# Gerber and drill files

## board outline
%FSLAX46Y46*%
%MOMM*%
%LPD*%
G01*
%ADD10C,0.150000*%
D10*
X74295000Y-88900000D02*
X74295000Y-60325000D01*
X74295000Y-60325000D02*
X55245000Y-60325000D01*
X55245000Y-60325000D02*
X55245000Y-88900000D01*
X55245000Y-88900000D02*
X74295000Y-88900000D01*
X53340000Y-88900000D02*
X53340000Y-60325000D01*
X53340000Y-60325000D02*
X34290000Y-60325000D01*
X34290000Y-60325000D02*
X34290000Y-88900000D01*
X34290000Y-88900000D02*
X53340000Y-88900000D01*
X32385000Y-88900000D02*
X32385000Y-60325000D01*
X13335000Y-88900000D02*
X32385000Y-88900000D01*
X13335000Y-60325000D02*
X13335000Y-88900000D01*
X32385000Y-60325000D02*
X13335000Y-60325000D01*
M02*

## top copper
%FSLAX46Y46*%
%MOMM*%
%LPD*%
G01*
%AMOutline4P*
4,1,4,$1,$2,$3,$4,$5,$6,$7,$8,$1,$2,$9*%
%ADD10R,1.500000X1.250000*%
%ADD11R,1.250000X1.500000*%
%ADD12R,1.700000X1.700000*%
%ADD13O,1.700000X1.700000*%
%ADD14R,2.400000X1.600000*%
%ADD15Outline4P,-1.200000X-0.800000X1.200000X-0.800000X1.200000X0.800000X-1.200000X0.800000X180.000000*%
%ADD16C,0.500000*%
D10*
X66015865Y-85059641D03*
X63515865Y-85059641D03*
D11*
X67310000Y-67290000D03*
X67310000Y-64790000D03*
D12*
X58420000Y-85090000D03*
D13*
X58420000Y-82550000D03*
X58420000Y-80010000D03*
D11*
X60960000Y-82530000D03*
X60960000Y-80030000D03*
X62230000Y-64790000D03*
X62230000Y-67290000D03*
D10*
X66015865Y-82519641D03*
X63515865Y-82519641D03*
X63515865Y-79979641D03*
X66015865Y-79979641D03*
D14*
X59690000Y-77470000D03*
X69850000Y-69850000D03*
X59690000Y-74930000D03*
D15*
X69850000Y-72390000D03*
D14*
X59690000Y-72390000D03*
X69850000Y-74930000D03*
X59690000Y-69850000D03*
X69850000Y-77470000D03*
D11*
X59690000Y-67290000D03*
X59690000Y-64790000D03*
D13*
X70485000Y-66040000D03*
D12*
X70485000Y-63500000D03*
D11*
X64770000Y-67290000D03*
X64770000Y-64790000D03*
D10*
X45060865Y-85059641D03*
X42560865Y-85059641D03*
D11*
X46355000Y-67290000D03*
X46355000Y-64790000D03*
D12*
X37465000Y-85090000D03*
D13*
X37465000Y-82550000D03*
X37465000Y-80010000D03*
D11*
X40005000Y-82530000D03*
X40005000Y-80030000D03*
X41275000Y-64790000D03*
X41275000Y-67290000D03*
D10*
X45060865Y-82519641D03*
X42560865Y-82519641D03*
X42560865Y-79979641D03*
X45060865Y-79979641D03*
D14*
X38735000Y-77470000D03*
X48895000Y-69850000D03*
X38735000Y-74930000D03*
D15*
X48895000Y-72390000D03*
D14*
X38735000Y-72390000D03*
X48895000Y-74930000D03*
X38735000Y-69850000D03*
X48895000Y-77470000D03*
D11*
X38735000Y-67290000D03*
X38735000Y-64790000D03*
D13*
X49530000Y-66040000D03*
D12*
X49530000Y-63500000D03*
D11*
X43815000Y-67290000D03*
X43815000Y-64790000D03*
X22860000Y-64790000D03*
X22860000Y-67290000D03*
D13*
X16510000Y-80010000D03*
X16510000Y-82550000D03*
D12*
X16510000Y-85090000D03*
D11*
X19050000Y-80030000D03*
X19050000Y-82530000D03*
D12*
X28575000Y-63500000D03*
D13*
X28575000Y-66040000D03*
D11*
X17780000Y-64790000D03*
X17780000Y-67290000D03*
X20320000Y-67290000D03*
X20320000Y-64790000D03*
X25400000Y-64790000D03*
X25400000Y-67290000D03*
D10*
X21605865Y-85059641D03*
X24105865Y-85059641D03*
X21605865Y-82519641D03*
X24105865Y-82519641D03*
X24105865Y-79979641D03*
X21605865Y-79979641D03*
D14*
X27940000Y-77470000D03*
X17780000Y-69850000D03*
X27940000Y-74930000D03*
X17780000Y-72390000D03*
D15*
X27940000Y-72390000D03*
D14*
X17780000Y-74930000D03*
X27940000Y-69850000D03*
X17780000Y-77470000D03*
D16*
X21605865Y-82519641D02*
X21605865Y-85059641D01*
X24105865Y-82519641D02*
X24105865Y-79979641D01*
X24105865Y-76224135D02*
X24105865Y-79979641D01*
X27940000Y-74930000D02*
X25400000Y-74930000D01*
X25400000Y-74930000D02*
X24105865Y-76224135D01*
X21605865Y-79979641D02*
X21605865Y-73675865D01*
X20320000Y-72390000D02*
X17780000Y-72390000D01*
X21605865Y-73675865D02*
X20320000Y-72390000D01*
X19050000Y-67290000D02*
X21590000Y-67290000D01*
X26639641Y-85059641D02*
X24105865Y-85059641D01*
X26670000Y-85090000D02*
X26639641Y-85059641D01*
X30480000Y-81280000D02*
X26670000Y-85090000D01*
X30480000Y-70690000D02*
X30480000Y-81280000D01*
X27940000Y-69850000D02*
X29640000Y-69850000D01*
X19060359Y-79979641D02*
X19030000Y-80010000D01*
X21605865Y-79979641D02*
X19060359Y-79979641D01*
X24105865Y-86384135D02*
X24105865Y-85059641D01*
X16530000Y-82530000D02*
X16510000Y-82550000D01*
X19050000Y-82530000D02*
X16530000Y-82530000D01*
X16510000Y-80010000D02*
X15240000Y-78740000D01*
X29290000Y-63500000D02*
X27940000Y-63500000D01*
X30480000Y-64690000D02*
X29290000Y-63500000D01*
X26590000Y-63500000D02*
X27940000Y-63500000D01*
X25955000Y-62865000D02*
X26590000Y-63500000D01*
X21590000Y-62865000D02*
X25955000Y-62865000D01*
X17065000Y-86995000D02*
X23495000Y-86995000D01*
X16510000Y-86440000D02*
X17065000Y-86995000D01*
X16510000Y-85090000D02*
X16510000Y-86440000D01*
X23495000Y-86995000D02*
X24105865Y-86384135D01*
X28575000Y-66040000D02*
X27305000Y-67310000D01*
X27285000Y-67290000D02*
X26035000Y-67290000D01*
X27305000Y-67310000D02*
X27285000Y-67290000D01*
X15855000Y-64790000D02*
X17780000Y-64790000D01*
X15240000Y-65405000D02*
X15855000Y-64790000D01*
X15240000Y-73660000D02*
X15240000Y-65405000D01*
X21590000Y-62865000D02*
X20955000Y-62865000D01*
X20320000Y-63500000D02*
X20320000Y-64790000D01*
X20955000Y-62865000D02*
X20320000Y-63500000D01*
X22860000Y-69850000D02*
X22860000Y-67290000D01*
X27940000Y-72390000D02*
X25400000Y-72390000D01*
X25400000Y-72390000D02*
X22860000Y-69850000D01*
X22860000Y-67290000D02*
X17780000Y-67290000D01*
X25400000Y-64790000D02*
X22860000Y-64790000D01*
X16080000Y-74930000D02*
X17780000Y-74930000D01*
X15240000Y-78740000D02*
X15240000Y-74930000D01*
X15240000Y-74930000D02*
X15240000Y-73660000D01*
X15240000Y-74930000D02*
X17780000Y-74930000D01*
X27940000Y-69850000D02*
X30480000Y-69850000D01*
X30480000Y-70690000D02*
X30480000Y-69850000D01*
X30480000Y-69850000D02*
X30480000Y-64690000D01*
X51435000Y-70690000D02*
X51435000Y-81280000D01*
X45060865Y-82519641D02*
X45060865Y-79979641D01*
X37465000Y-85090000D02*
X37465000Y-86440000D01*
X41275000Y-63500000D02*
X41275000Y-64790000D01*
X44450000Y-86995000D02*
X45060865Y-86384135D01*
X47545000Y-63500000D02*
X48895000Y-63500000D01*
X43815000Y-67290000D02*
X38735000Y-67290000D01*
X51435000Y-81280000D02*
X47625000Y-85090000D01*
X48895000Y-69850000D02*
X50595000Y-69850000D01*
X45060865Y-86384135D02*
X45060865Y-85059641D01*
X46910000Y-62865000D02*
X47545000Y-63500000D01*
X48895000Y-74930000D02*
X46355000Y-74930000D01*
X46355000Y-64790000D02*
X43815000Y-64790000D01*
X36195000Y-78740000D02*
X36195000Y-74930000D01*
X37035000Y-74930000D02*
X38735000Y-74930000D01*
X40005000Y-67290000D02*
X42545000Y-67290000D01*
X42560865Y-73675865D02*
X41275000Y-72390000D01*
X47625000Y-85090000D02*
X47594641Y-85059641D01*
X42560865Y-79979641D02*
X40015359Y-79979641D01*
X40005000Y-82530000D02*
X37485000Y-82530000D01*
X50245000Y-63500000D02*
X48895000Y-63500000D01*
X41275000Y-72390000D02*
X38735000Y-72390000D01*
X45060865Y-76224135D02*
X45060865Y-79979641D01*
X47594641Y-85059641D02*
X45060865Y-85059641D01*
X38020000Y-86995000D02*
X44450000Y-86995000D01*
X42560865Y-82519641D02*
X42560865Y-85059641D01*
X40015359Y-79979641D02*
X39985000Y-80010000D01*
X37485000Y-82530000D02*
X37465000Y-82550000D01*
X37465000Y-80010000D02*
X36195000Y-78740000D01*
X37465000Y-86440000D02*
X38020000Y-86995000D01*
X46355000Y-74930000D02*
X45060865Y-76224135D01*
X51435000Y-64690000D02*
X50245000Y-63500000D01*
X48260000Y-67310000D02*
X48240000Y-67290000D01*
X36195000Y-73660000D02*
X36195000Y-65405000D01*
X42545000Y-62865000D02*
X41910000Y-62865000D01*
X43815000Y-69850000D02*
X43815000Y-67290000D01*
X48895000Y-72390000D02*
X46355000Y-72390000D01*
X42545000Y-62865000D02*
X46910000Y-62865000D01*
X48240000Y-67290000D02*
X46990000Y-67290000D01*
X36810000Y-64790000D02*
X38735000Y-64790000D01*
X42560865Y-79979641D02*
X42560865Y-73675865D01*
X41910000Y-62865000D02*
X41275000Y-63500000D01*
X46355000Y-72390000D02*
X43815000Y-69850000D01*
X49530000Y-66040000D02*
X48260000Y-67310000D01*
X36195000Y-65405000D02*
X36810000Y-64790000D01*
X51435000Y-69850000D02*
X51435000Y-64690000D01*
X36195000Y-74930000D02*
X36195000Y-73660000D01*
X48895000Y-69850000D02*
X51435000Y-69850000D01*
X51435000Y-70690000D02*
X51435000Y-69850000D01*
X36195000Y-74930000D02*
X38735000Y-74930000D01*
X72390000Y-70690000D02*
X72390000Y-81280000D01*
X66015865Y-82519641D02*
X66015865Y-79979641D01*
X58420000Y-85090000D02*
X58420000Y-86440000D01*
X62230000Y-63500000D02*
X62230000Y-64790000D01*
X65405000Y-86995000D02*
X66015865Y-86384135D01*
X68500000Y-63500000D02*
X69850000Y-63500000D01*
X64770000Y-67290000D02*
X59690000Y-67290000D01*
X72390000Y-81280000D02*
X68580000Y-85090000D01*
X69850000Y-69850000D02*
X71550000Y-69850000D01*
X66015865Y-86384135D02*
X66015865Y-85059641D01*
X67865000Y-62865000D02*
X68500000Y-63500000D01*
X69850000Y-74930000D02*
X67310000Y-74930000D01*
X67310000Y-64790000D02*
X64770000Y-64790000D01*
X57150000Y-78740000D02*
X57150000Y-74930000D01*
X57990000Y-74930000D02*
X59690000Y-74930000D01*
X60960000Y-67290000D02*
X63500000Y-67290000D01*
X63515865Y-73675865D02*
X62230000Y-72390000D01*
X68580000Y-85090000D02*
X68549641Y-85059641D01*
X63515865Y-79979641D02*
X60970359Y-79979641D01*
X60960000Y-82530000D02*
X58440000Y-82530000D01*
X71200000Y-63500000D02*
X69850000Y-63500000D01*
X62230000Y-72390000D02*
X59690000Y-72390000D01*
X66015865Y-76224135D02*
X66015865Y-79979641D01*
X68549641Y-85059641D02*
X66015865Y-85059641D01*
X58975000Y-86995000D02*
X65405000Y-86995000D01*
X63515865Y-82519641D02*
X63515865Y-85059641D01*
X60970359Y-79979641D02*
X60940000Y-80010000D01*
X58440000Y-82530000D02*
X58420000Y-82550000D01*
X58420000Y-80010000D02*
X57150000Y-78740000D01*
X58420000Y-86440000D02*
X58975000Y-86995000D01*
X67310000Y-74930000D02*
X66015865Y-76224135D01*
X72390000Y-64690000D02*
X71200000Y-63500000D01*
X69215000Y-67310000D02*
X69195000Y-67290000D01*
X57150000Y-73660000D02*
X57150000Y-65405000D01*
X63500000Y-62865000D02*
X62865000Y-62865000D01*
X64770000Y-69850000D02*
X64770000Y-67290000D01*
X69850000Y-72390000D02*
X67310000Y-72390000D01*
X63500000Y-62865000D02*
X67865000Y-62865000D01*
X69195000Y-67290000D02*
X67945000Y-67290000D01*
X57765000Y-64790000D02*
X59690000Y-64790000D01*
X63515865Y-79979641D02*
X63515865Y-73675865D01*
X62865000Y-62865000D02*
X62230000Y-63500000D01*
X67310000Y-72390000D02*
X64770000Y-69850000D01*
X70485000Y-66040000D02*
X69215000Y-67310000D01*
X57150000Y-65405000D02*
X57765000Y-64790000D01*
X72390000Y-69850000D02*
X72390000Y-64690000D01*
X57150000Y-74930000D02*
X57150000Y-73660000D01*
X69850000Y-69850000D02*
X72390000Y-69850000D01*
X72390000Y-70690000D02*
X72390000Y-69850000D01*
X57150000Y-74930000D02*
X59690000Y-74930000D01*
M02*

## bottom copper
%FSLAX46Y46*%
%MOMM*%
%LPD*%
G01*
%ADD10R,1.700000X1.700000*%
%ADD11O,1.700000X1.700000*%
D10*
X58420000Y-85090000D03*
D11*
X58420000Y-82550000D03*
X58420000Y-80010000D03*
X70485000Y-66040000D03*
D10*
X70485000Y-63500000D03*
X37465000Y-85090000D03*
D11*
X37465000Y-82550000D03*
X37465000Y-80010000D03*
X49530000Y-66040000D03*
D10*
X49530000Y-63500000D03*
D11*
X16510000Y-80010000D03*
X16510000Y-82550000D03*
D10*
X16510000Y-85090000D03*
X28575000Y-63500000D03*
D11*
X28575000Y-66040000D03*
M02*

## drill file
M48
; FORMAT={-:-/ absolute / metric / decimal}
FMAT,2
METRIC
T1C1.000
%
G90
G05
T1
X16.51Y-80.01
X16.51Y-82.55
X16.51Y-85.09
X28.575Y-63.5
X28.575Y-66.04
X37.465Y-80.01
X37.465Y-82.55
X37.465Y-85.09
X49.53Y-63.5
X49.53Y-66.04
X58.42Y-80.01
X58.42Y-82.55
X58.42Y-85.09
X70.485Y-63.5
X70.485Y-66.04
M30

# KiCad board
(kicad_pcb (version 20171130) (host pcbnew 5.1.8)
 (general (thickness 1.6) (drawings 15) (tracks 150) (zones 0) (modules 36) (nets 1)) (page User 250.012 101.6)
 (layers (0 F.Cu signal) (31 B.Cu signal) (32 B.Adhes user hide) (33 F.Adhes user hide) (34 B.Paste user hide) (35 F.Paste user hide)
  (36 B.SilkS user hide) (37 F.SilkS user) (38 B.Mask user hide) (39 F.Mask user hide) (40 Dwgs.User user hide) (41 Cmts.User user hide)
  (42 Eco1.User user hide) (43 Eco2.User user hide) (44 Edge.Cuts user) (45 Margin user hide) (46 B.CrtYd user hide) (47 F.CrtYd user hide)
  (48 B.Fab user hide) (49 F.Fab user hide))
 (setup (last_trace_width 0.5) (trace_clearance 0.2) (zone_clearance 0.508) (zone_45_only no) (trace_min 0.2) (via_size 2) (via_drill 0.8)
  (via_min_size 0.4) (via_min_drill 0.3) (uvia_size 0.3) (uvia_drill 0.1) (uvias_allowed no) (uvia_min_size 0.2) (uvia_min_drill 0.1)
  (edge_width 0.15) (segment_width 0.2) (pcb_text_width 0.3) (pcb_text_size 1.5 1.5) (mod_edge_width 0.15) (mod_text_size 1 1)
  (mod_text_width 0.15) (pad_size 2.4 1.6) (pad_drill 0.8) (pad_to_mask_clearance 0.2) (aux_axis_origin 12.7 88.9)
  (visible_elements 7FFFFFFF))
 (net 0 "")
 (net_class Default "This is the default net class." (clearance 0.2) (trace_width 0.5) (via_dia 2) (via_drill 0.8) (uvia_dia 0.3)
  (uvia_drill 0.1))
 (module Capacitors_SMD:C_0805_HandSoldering (layer F.Cu) (at 64.765865 85.059641 180)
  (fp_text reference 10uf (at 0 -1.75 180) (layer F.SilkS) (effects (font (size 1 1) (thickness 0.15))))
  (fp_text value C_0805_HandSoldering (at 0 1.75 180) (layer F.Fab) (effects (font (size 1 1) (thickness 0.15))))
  (pad 1 smd rect (at -1.25 0 180) (size 1.5 1.25) (layers F.Cu F.Paste F.Mask))
  (pad 2 smd rect (at 1.25 0 180) (size 1.5 1.25) (layers F.Cu F.Paste F.Mask)))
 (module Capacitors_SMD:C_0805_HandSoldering (layer F.Cu) (at 67.31 66.04 270)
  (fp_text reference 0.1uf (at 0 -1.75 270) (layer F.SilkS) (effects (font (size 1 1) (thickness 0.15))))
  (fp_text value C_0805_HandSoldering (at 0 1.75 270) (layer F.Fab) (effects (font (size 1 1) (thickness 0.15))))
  (pad 2 smd rect (at 1.25 0 270) (size 1.5 1.25) (layers F.Cu F.Paste F.Mask))
  (pad 1 smd rect (at -1.25 0 270) (size 1.5 1.25) (layers F.Cu F.Paste F.Mask)))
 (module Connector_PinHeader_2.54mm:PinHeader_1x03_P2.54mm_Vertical (layer F.Cu) (at 58.42 85.09 180)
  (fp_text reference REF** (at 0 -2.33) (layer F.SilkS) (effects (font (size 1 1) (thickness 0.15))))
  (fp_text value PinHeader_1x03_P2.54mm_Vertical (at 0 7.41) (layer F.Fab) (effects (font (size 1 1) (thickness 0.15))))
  (pad 1 thru_hole rect (at 0 0 180) (size 1.7 1.7) (drill 1) (layers *.Cu *.Mask))
  (pad 2 thru_hole oval (at 0 2.54 180) (size 1.7 1.7) (drill 1) (layers *.Cu *.Mask))
  (pad 3 thru_hole oval (at 0 5.08 180) (size 1.7 1.7) (drill 1) (layers *.Cu *.Mask)))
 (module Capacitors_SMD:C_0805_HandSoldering (layer F.Cu) (at 60.96 81.28 270)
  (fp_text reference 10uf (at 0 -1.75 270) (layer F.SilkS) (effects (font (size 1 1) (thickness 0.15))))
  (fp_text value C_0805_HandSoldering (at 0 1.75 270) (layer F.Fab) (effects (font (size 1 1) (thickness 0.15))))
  (pad 2 smd rect (at 1.25 0 270) (size 1.5 1.25) (layers F.Cu F.Paste F.Mask))
  (pad 1 smd rect (at -1.25 0 270) (size 1.5 1.25) (layers F.Cu F.Paste F.Mask)))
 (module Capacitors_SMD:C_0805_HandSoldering (layer F.Cu) (at 62.23 66.04 270)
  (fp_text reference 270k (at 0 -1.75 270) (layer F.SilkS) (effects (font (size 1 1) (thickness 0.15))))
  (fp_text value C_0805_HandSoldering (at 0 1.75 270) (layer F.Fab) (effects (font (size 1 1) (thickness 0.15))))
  (pad 1 smd rect (at -1.25 0 270) (size 1.5 1.25) (layers F.Cu F.Paste F.Mask))
  (pad 2 smd rect (at 1.25 0 270) (size 1.5 1.25) (layers F.Cu F.Paste F.Mask)))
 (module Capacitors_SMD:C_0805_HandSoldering (layer F.Cu) (at 64.765865 82.519641 180)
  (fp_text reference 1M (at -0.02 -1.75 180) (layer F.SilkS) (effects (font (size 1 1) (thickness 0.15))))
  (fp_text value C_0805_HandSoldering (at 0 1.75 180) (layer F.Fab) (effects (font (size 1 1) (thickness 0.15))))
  (pad 1 smd rect (at -1.25 0 180) (size 1.5 1.25) (layers F.Cu F.Paste F.Mask))
  (pad 2 smd rect (at 1.25 0 180) (size 1.5 1.25) (layers F.Cu F.Paste F.Mask)))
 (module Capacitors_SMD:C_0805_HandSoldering (layer F.Cu) (at 64.765865 79.979641 180)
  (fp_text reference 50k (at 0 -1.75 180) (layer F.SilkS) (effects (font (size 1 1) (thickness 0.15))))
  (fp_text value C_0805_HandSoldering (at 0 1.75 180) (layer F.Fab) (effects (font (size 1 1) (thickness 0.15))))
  (pad 2 smd rect (at 1.25 0 180) (size 1.5 1.25) (layers F.Cu F.Paste F.Mask))
  (pad 1 smd rect (at -1.25 0 180) (size 1.5 1.25) (layers F.Cu F.Paste F.Mask)))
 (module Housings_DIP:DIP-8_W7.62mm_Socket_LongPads (layer F.Cu) (at 68.58 77.47 180)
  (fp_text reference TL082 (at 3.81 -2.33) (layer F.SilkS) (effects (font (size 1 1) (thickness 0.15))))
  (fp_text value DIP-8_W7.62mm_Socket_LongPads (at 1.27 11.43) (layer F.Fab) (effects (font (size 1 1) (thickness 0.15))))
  (pad 8 smd rect (at 8.89 0 180) (size 2.4 1.6) (layers F.Cu F.Paste F.Mask))
  (pad 4 smd rect (at -1.27 7.62 180) (size 2.4 1.6) (layers F.Cu F.Paste F.Mask))
  (pad 7 smd rect (at 8.89 2.54 180) (size 2.4 1.6) (layers F.Cu F.Paste F.Mask))
  (pad 3 smd trapezoid (at -1.27 5.08 180) (size 2.4 1.6) (layers F.Cu F.Paste F.Mask))
  (pad 6 smd rect (at 8.89 5.08 180) (size 2.4 1.6) (layers F.Cu F.Paste F.Mask))
  (pad 2 smd rect (at -1.27 2.54 180) (size 2.4 1.6) (layers F.Cu F.Paste F.Mask))
  (pad 5 smd rect (at 8.89 7.62 180) (size 2.4 1.6) (layers F.Cu F.Paste F.Mask))
  (pad 1 smd rect (at -1.27 0 180) (size 2.4 1.6) (layers F.Cu F.Paste F.Mask)))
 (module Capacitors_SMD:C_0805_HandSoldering (layer F.Cu) (at 59.69 66.04 270)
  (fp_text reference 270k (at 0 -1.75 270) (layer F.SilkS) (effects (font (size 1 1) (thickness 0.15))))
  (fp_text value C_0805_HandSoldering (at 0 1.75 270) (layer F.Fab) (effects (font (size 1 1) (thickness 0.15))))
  (pad 2 smd rect (at 1.25 0 270) (size 1.5 1.25) (layers F.Cu F.Paste F.Mask))
  (pad 1 smd rect (at -1.25 0 270) (size 1.5 1.25) (layers F.Cu F.Paste F.Mask)))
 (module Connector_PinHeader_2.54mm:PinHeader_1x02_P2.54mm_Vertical (layer F.Cu) (at 70.485 63.5)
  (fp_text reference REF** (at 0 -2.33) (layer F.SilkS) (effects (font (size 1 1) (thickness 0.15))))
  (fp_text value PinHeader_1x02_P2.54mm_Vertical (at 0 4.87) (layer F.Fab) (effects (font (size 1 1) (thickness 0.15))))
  (pad 2 thru_hole oval (at 0 2.54) (size 1.7 1.7) (drill 1) (layers *.Cu *.Mask))
  (pad 1 thru_hole rect (at 0 0) (size 1.7 1.7) (drill 1) (layers *.Cu *.Mask)))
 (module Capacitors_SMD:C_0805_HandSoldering (layer F.Cu) (at 64.77 66.04 270)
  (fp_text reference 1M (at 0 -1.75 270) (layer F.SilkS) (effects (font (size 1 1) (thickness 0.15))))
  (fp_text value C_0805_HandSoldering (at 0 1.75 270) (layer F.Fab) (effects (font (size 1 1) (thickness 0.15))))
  (pad 2 smd rect (at 1.25 0 270) (size 1.5 1.25) (layers F.Cu F.Paste F.Mask))
  (pad 1 smd rect (at -1.25 0 270) (size 1.5 1.25) (layers F.Cu F.Paste F.Mask)))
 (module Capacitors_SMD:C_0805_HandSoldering (layer F.Cu) (at 43.810865 85.059641 180)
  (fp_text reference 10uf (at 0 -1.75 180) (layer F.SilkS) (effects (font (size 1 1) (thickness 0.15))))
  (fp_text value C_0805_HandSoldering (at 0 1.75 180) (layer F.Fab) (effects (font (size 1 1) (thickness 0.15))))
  (pad 1 smd rect (at -1.25 0 180) (size 1.5 1.25) (layers F.Cu F.Paste F.Mask))
  (pad 2 smd rect (at 1.25 0 180) (size 1.5 1.25) (layers F.Cu F.Paste F.Mask)))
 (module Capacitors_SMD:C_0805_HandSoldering (layer F.Cu) (at 46.355 66.04 270)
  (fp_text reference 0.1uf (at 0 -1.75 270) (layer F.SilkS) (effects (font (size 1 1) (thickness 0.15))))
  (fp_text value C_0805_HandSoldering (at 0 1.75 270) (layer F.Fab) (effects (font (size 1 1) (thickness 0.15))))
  (pad 2 smd rect (at 1.25 0 270) (size 1.5 1.25) (layers F.Cu F.Paste F.Mask))
  (pad 1 smd rect (at -1.25 0 270) (size 1.5 1.25) (layers F.Cu F.Paste F.Mask)))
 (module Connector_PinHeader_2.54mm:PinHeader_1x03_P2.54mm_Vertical (layer F.Cu) (at 37.465 85.09 180)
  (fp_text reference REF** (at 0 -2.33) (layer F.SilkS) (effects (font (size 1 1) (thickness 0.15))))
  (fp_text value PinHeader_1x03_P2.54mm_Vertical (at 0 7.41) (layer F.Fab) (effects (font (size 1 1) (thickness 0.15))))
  (pad 1 thru_hole rect (at 0 0 180) (size 1.7 1.7) (drill 1) (layers *.Cu *.Mask))
  (pad 2 thru_hole oval (at 0 2.54 180) (size 1.7 1.7) (drill 1) (layers *.Cu *.Mask))
  (pad 3 thru_hole oval (at 0 5.08 180) (size 1.7 1.7) (drill 1) (layers *.Cu *.Mask)))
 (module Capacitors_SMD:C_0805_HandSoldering (layer F.Cu) (at 40.005 81.28 270)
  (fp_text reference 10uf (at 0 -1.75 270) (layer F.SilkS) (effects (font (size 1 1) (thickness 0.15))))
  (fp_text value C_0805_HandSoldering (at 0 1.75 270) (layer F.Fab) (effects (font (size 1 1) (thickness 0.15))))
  (pad 2 smd rect (at 1.25 0 270) (size 1.5 1.25) (layers F.Cu F.Paste F.Mask))
  (pad 1 smd rect (at -1.25 0 270) (size 1.5 1.25) (layers F.Cu F.Paste F.Mask)))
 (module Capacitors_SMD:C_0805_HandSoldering (layer F.Cu) (at 41.275 66.04 270)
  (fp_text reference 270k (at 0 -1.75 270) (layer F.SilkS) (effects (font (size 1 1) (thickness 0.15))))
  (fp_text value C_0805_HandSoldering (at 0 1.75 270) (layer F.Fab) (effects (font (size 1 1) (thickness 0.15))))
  (pad 1 smd rect (at -1.25 0 270) (size 1.5 1.25) (layers F.Cu F.Paste F.Mask))
  (pad 2 smd rect (at 1.25 0 270) (size 1.5 1.25) (layers F.Cu F.Paste F.Mask)))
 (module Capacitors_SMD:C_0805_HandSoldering (layer F.Cu) (at 43.810865 82.519641 180)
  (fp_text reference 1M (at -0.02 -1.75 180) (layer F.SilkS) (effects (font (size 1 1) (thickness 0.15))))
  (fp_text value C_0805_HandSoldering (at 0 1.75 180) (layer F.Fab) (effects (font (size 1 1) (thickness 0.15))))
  (pad 1 smd rect (at -1.25 0 180) (size 1.5 1.25) (layers F.Cu F.Paste F.Mask))
  (pad 2 smd rect (at 1.25 0 180) (size 1.5 1.25) (layers F.Cu F.Paste F.Mask)))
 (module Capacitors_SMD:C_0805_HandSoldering (layer F.Cu) (at 43.810865 79.979641 180)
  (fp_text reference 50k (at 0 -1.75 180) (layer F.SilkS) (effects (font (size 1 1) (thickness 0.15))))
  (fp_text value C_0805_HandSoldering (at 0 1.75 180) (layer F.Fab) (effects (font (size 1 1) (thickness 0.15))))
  (pad 2 smd rect (at 1.25 0 180) (size 1.5 1.25) (layers F.Cu F.Paste F.Mask))
  (pad 1 smd rect (at -1.25 0 180) (size 1.5 1.25) (layers F.Cu F.Paste F.Mask)))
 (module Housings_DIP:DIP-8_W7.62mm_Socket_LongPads (layer F.Cu) (at 47.625 77.47 180)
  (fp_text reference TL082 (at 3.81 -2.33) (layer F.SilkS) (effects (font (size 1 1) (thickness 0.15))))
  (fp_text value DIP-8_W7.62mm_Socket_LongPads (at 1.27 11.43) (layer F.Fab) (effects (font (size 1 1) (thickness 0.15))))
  (pad 8 smd rect (at 8.89 0 180) (size 2.4 1.6) (layers F.Cu F.Paste F.Mask))
  (pad 4 smd rect (at -1.27 7.62 180) (size 2.4 1.6) (layers F.Cu F.Paste F.Mask))
  (pad 7 smd rect (at 8.89 2.54 180) (size 2.4 1.6) (layers F.Cu F.Paste F.Mask))
  (pad 3 smd trapezoid (at -1.27 5.08 180) (size 2.4 1.6) (layers F.Cu F.Paste F.Mask))
  (pad 6 smd rect (at 8.89 5.08 180) (size 2.4 1.6) (layers F.Cu F.Paste F.Mask))
  (pad 2 smd rect (at -1.27 2.54 180) (size 2.4 1.6) (layers F.Cu F.Paste F.Mask))
  (pad 5 smd rect (at 8.89 7.62 180) (size 2.4 1.6) (layers F.Cu F.Paste F.Mask))
  (pad 1 smd rect (at -1.27 0 180) (size 2.4 1.6) (layers F.Cu F.Paste F.Mask)))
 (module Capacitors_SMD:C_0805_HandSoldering (layer F.Cu) (at 38.735 66.04 270)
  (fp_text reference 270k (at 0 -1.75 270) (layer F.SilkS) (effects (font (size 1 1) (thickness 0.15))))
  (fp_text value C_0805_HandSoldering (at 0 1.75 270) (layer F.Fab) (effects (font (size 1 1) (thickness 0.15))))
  (pad 2 smd rect (at 1.25 0 270) (size 1.5 1.25) (layers F.Cu F.Paste F.Mask))
  (pad 1 smd rect (at -1.25 0 270) (size 1.5 1.25) (layers F.Cu F.Paste F.Mask)))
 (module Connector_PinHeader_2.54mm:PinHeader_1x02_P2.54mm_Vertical (layer F.Cu) (at 49.53 63.5)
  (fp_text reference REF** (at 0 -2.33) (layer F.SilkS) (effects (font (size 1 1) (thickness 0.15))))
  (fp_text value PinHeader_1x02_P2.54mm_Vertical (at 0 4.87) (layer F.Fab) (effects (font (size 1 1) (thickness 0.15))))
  (pad 2 thru_hole oval (at 0 2.54) (size 1.7 1.7) (drill 1) (layers *.Cu *.Mask))
  (pad 1 thru_hole rect (at 0 0) (size 1.7 1.7) (drill 1) (layers *.Cu *.Mask)))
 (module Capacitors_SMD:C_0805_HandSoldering (layer F.Cu) (at 43.815 66.04 270)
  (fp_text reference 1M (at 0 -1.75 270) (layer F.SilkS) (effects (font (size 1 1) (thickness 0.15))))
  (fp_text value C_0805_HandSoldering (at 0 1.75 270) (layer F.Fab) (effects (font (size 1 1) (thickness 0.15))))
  (pad 2 smd rect (at 1.25 0 270) (size 1.5 1.25) (layers F.Cu F.Paste F.Mask))
  (pad 1 smd rect (at -1.25 0 270) (size 1.5 1.25) (layers F.Cu F.Paste F.Mask)))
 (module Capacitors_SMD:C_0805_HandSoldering (layer F.Cu) (at 22.86 66.04 270)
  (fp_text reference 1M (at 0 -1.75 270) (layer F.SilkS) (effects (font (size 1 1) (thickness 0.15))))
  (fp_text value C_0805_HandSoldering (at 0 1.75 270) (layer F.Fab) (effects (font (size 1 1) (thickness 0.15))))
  (pad 1 smd rect (at -1.25 0 270) (size 1.5 1.25) (layers F.Cu F.Paste F.Mask))
  (pad 2 smd rect (at 1.25 0 270) (size 1.5 1.25) (layers F.Cu F.Paste F.Mask)))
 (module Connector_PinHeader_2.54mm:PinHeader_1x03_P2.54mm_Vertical (layer F.Cu) (at 16.51 85.09 180)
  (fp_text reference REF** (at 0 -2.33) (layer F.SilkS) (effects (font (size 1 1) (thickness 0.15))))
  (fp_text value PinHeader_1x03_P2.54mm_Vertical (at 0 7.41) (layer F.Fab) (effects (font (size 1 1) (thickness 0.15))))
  (pad 3 thru_hole oval (at 0 5.08 180) (size 1.7 1.7) (drill 1) (layers *.Cu *.Mask))
  (pad 2 thru_hole oval (at 0 2.54 180) (size 1.7 1.7) (drill 1) (layers *.Cu *.Mask))
  (pad 1 thru_hole rect (at 0 0 180) (size 1.7 1.7) (drill 1) (layers *.Cu *.Mask)))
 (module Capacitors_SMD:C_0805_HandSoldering (layer F.Cu) (at 19.05 81.28 270)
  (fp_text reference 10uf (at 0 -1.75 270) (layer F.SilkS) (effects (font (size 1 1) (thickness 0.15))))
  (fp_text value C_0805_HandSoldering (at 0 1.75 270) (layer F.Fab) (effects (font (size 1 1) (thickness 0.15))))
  (pad 1 smd rect (at -1.25 0 270) (size 1.5 1.25) (layers F.Cu F.Paste F.Mask))
  (pad 2 smd rect (at 1.25 0 270) (size 1.5 1.25) (layers F.Cu F.Paste F.Mask)))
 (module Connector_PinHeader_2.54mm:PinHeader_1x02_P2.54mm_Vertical (layer F.Cu) (at 28.575 63.5)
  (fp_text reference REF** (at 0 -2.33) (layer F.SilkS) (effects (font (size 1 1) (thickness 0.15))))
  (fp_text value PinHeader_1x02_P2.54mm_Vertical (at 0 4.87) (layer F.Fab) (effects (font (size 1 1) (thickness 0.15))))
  (pad 1 thru_hole rect (at 0 0) (size 1.7 1.7) (drill 1) (layers *.Cu *.Mask))
  (pad 2 thru_hole oval (at 0 2.54) (size 1.7 1.7) (drill 1) (layers *.Cu *.Mask)))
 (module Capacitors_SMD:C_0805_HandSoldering (layer F.Cu) (at 17.78 66.04 270)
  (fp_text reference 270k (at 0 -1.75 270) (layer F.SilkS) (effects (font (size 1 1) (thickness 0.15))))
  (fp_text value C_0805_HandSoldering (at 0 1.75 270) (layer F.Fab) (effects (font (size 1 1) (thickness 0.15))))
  (pad 1 smd rect (at -1.25 0 270) (size 1.5 1.25) (layers F.Cu F.Paste F.Mask))
  (pad 2 smd rect (at 1.25 0 270) (size 1.5 1.25) (layers F.Cu F.Paste F.Mask)))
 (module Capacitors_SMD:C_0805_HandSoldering (layer F.Cu) (at 20.32 66.04 270)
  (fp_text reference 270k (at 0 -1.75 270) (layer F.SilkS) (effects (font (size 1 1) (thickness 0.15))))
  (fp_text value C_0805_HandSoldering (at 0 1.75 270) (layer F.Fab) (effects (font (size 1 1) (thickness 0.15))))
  (pad 2 smd rect (at 1.25 0 270) (size 1.5 1.25) (layers F.Cu F.Paste F.Mask))
  (pad 1 smd rect (at -1.25 0 270) (size 1.5 1.25) (layers F.Cu F.Paste F.Mask)))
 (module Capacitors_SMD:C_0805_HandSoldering (layer F.Cu) (at 25.4 66.04 270)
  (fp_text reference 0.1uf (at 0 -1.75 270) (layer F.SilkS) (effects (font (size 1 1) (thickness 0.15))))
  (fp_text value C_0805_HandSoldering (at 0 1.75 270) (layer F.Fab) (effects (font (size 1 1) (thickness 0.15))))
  (pad 1 smd rect (at -1.25 0 270) (size 1.5 1.25) (layers F.Cu F.Paste F.Mask))
  (pad 2 smd rect (at 1.25 0 270) (size 1.5 1.25) (layers F.Cu F.Paste F.Mask)))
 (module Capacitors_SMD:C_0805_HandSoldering (layer F.Cu) (at 22.855865 85.059641 180)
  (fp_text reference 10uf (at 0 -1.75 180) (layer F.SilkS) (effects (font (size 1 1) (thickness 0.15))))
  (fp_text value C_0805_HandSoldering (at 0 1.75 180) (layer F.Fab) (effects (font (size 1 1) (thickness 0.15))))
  (pad 2 smd rect (at 1.25 0 180) (size 1.5 1.25) (layers F.Cu F.Paste F.Mask))
  (pad 1 smd rect (at -1.25 0 180) (size 1.5 1.25) (layers F.Cu F.Paste F.Mask)))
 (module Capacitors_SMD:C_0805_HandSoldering (layer F.Cu) (at 22.855865 82.519641 180)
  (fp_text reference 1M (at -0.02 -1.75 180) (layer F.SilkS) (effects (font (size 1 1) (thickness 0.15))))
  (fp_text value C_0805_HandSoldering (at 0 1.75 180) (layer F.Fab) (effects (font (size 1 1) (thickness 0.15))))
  (pad 2 smd rect (at 1.25 0 180) (size 1.5 1.25) (layers F.Cu F.Paste F.Mask))
  (pad 1 smd rect (at -1.25 0 180) (size 1.5 1.25) (layers F.Cu F.Paste F.Mask)))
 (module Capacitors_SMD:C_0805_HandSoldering (layer F.Cu) (at 22.855865 79.979641 180)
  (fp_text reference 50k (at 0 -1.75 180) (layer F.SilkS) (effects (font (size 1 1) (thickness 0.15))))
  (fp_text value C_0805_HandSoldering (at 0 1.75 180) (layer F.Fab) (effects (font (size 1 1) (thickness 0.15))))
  (pad 1 smd rect (at -1.25 0 180) (size 1.5 1.25) (layers F.Cu F.Paste F.Mask))
  (pad 2 smd rect (at 1.25 0 180) (size 1.5 1.25) (layers F.Cu F.Paste F.Mask)))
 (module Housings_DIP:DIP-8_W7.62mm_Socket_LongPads (layer F.Cu) (at 26.67 77.47 180)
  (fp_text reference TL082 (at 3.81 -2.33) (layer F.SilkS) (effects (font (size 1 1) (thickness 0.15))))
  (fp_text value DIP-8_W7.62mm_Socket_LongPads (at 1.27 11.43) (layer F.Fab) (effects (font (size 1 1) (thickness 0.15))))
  (pad 1 smd rect (at -1.27 0 180) (size 2.4 1.6) (layers F.Cu F.Paste F.Mask))
  (pad 5 smd rect (at 8.89 7.62 180) (size 2.4 1.6) (layers F.Cu F.Paste F.Mask))
  (pad 2 smd rect (at -1.27 2.54 180) (size 2.4 1.6) (layers F.Cu F.Paste F.Mask))
  (pad 6 smd rect (at 8.89 5.08 180) (size 2.4 1.6) (layers F.Cu F.Paste F.Mask))
  (pad 3 smd trapezoid (at -1.27 5.08 180) (size 2.4 1.6) (layers F.Cu F.Paste F.Mask))
  (pad 7 smd rect (at 8.89 2.54 180) (size 2.4 1.6) (layers F.Cu F.Paste F.Mask))
  (pad 4 smd rect (at -1.27 7.62 180) (size 2.4 1.6) (layers F.Cu F.Paste F.Mask))
  (pad 8 smd rect (at 8.89 0 180) (size 2.4 1.6) (layers F.Cu F.Paste F.Mask)))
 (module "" (layer F.Cu) (at 111 64)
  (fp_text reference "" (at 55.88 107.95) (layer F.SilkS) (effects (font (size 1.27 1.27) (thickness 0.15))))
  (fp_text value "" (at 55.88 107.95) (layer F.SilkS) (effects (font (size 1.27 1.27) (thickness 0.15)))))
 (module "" (layer F.Cu) (at 116 67)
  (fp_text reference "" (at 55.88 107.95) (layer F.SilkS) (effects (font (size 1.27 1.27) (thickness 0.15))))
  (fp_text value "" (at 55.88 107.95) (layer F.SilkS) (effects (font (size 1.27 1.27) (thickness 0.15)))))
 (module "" (layer F.Cu) (at 99 74)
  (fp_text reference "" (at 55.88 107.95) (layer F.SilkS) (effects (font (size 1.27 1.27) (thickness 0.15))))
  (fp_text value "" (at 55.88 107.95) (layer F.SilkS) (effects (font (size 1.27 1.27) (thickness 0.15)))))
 (gr_line (start 74.295 88.9) (end 74.295 60.325) (layer Edge.Cuts) (width 0.15))
 (gr_line (start 74.295 60.325) (end 55.245 60.325) (layer Edge.Cuts) (width 0.15))
 (gr_line (start 55.245 60.325) (end 55.245 88.9) (layer Edge.Cuts) (width 0.15))
 (gr_line (start 55.245 88.9) (end 74.295 88.9) (layer Edge.Cuts) (width 0.15))
 (gr_line (start 53.34 88.9) (end 53.34 60.325) (layer Edge.Cuts) (width 0.15))
 (gr_line (start 53.34 60.325) (end 34.29 60.325) (layer Edge.Cuts) (width 0.15))
 (gr_line (start 34.29 60.325) (end 34.29 88.9) (layer Edge.Cuts) (width 0.15))
 (gr_line (start 34.29 88.9) (end 53.34 88.9) (layer Edge.Cuts) (width 0.15))
 (gr_line (start 32.385 88.9) (end 32.385 60.325) (layer Edge.Cuts) (width 0.15))
 (gr_line (start 13.335 88.9) (end 32.385 88.9) (layer Edge.Cuts) (width 0.15))
 (gr_line (start 13.335 60.325) (end 13.335 88.9) (layer Edge.Cuts) (width 0.15))
 (gr_line (start 32.385 60.325) (end 13.335 60.325) (layer Edge.Cuts) (width 0.15))
 (segment (start 21.605865 82.519641) (end 21.605865 85.059641) (width 0.5) (layer F.Cu) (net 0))
 (segment (start 24.105865 82.519641) (end 24.105865 79.979641) (width 0.5) (layer F.Cu) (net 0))
 (segment (start 24.105865 76.224135) (end 24.105865 79.979641) (width 0.5) (layer F.Cu) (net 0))
 (segment (start 27.94 74.93) (end 25.4 74.93) (width 0.5) (layer F.Cu) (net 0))
 (segment (start 25.4 74.93) (end 24.105865 76.224135) (width 0.5) (layer F.Cu) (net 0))
 (segment (start 21.605865 79.979641) (end 21.605865 73.675865) (width 0.5) (layer F.Cu) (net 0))
 (segment (start 20.32 72.39) (end 17.78 72.39) (width 0.5) (layer F.Cu) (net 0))
 (segment (start 21.605865 73.675865) (end 20.32 72.39) (width 0.5) (layer F.Cu) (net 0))
 (segment (start 19.05 67.29) (end 21.59 67.29) (width 0.5) (layer F.Cu) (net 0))
 (segment (start 26.639641 85.059641) (end 24.105865 85.059641) (width 0.5) (layer F.Cu) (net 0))
 (segment (start 26.67 85.09) (end 26.639641 85.059641) (width 0.5) (layer F.Cu) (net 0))
 (segment (start 30.48 81.28) (end 26.67 85.09) (width 0.5) (layer F.Cu) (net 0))
 (segment (start 30.48 70.69) (end 30.48 81.28) (width 0.5) (layer F.Cu) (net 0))
 (segment (start 27.94 69.85) (end 29.64 69.85) (width 0.5) (layer F.Cu) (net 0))
 (segment (start 19.060359 79.979641) (end 19.03 80.01) (width 0.5) (layer F.Cu) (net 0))
 (segment (start 21.605865 79.979641) (end 19.060359 79.979641) (width 0.5) (layer F.Cu) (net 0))
 (segment (start 24.105865 86.384135) (end 24.105865 85.059641) (width 0.5) (layer F.Cu) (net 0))
 (segment (start 16.53 82.53) (end 16.51 82.55) (width 0.5) (layer F.Cu) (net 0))
 (segment (start 19.05 82.53) (end 16.53 82.53) (width 0.5) (layer F.Cu) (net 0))
 (segment (start 16.51 80.01) (end 15.24 78.74) (width 0.5) (layer F.Cu) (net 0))
 (segment (start 29.29 63.5) (end 27.94 63.5) (width 0.5) (layer F.Cu) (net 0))
 (segment (start 30.48 64.69) (end 29.29 63.5) (width 0.5) (layer F.Cu) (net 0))
 (segment (start 26.59 63.5) (end 27.94 63.5) (width 0.5) (layer F.Cu) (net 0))
 (segment (start 25.955 62.865) (end 26.59 63.5) (width 0.5) (layer F.Cu) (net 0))
 (segment (start 21.59 62.865) (end 25.955 62.865) (width 0.5) (layer F.Cu) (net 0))
 (segment (start 17.065 86.995) (end 23.495 86.995) (width 0.5) (layer F.Cu) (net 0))
 (segment (start 16.51 86.44) (end 17.065 86.995) (width 0.5) (layer F.Cu) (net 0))
 (segment (start 16.51 85.09) (end 16.51 86.44) (width 0.5) (layer F.Cu) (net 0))
 (segment (start 23.495 86.995) (end 24.105865 86.384135) (width 0.5) (layer F.Cu) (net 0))
 (segment (start 28.575 66.04) (end 27.305 67.31) (width 0.5) (layer F.Cu) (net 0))
 (segment (start 27.285 67.29) (end 26.035 67.29) (width 0.5) (layer F.Cu) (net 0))
 (segment (start 27.305 67.31) (end 27.285 67.29) (width 0.5) (layer F.Cu) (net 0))
 (segment (start 15.855 64.79) (end 17.78 64.79) (width 0.5) (layer F.Cu) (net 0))
 (segment (start 15.24 65.405) (end 15.855 64.79) (width 0.5) (layer F.Cu) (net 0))
 (segment (start 15.24 73.66) (end 15.24 65.405) (width 0.5) (layer F.Cu) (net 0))
 (segment (start 21.59 62.865) (end 20.955 62.865) (width 0.5) (layer F.Cu) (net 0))
 (segment (start 20.32 63.5) (end 20.32 64.79) (width 0.5) (layer F.Cu) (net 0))
 (segment (start 20.955 62.865) (end 20.32 63.5) (width 0.5) (layer F.Cu) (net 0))
 (segment (start 22.86 69.85) (end 22.86 67.29) (width 0.5) (layer F.Cu) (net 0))
 (segment (start 27.94 72.39) (end 25.4 72.39) (width 0.5) (layer F.Cu) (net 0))
 (segment (start 25.4 72.39) (end 22.86 69.85) (width 0.5) (layer F.Cu) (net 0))
 (segment (start 22.86 67.29) (end 17.78 67.29) (width 0.5) (layer F.Cu) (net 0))
 (segment (start 25.4 64.79) (end 22.86 64.79) (width 0.5) (layer F.Cu) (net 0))
 (segment (start 16.08 74.93) (end 17.78 74.93) (width 0.5) (layer F.Cu) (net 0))
 (segment (start 15.24 78.74) (end 15.24 74.93) (width 0.5) (layer F.Cu) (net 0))
 (segment (start 15.24 74.93) (end 15.24 73.66) (width 0.5) (layer F.Cu) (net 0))
 (segment (start 15.24 74.93) (end 17.78 74.93) (width 0.5) (layer F.Cu) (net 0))
 (segment (start 27.94 69.85) (end 30.48 69.85) (width 0.5) (layer F.Cu) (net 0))
 (segment (start 30.48 70.69) (end 30.48 69.85) (width 0.5) (layer F.Cu) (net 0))
 (segment (start 30.48 69.85) (end 30.48 64.69) (width 0.5) (layer F.Cu) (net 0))
 (segment (start 51.435 70.69) (end 51.435 81.28) (width 0.5) (layer F.Cu) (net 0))
 (segment (start 45.060865 82.519641) (end 45.060865 79.979641) (width 0.5) (layer F.Cu) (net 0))
 (segment (start 37.465 85.09) (end 37.465 86.44) (width 0.5) (layer F.Cu) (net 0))
 (segment (start 41.275 63.5) (end 41.275 64.79) (width 0.5) (layer F.Cu) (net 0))
 (segment (start 44.45 86.995) (end 45.060865 86.384135) (width 0.5) (layer F.Cu) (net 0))
 (segment (start 47.545 63.5) (end 48.895 63.5) (width 0.5) (layer F.Cu) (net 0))
 (segment (start 43.815 67.29) (end 38.735 67.29) (width 0.5) (layer F.Cu) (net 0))
 (segment (start 51.435 81.28) (end 47.625 85.09) (width 0.5) (layer F.Cu) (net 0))
 (segment (start 48.895 69.85) (end 50.595 69.85) (width 0.5) (layer F.Cu) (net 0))
 (segment (start 45.060865 86.384135) (end 45.060865 85.059641) (width 0.5) (layer F.Cu) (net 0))
 (segment (start 46.91 62.865) (end 47.545 63.5) (width 0.5) (layer F.Cu) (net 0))
 (segment (start 48.895 74.93) (end 46.355 74.93) (width 0.5) (layer F.Cu) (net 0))
 (segment (start 46.355 64.79) (end 43.815 64.79) (width 0.5) (layer F.Cu) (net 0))
 (segment (start 36.195 78.74) (end 36.195 74.93) (width 0.5) (layer F.Cu) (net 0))
 (segment (start 37.035 74.93) (end 38.735 74.93) (width 0.5) (layer F.Cu) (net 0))
 (segment (start 40.005 67.29) (end 42.545 67.29) (width 0.5) (layer F.Cu) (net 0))
 (segment (start 42.560865 73.675865) (end 41.275 72.39) (width 0.5) (layer F.Cu) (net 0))
 (segment (start 47.625 85.09) (end 47.594641 85.059641) (width 0.5) (layer F.Cu) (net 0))
 (segment (start 42.560865 79.979641) (end 40.015359 79.979641) (width 0.5) (layer F.Cu) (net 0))
 (segment (start 40.005 82.53) (end 37.485 82.53) (width 0.5) (layer F.Cu) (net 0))
 (segment (start 50.245 63.5) (end 48.895 63.5) (width 0.5) (layer F.Cu) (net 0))
 (segment (start 41.275 72.39) (end 38.735 72.39) (width 0.5) (layer F.Cu) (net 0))
 (segment (start 45.060865 76.224135) (end 45.060865 79.979641) (width 0.5) (layer F.Cu) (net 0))
 (segment (start 47.594641 85.059641) (end 45.060865 85.059641) (width 0.5) (layer F.Cu) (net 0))
 (segment (start 38.02 86.995) (end 44.45 86.995) (width 0.5) (layer F.Cu) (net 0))
 (segment (start 42.560865 82.519641) (end 42.560865 85.059641) (width 0.5) (layer F.Cu) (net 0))
 (segment (start 40.015359 79.979641) (end 39.985 80.01) (width 0.5) (layer F.Cu) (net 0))
 (segment (start 37.485 82.53) (end 37.465 82.55) (width 0.5) (layer F.Cu) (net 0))
 (segment (start 37.465 80.01) (end 36.195 78.74) (width 0.5) (layer F.Cu) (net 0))
 (segment (start 37.465 86.44) (end 38.02 86.995) (width 0.5) (layer F.Cu) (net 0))
 (segment (start 46.355 74.93) (end 45.060865 76.224135) (width 0.5) (layer F.Cu) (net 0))
 (segment (start 51.435 64.69) (end 50.245 63.5) (width 0.5) (layer F.Cu) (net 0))
 (segment (start 48.26 67.31) (end 48.24 67.29) (width 0.5) (layer F.Cu) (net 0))
 (segment (start 36.195 73.66) (end 36.195 65.405) (width 0.5) (layer F.Cu) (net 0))
 (segment (start 42.545 62.865) (end 41.91 62.865) (width 0.5) (layer F.Cu) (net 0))
 (segment (start 43.815 69.85) (end 43.815 67.29) (width 0.5) (layer F.Cu) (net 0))
 (segment (start 48.895 72.39) (end 46.355 72.39) (width 0.5) (layer F.Cu) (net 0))
 (segment (start 42.545 62.865) (end 46.91 62.865) (width 0.5) (layer F.Cu) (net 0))
 (segment (start 48.24 67.29) (end 46.99 67.29) (width 0.5) (layer F.Cu) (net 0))
 (segment (start 36.81 64.79) (end 38.735 64.79) (width 0.5) (layer F.Cu) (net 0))
 (segment (start 42.560865 79.979641) (end 42.560865 73.675865) (width 0.5) (layer F.Cu) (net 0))
 (segment (start 41.91 62.865) (end 41.275 63.5) (width 0.5) (layer F.Cu) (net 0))
 (segment (start 46.355 72.39) (end 43.815 69.85) (width 0.5) (layer F.Cu) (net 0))
 (segment (start 49.53 66.04) (end 48.26 67.31) (width 0.5) (layer F.Cu) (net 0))
 (segment (start 36.195 65.405) (end 36.81 64.79) (width 0.5) (layer F.Cu) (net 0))
 (segment (start 51.435 69.85) (end 51.435 64.69) (width 0.5) (layer F.Cu) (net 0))
 (segment (start 36.195 74.93) (end 36.195 73.66) (width 0.5) (layer F.Cu) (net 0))
 (segment (start 48.895 69.85) (end 51.435 69.85) (width 0.5) (layer F.Cu) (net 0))
 (segment (start 51.435 70.69) (end 51.435 69.85) (width 0.5) (layer F.Cu) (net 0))
 (segment (start 36.195 74.93) (end 38.735 74.93) (width 0.5) (layer F.Cu) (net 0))
 (segment (start 72.39 70.69) (end 72.39 81.28) (width 0.5) (layer F.Cu) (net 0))
 (segment (start 66.015865 82.519641) (end 66.015865 79.979641) (width 0.5) (layer F.Cu) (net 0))
 (segment (start 58.42 85.09) (end 58.42 86.44) (width 0.5) (layer F.Cu) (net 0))
 (segment (start 62.23 63.5) (end 62.23 64.79) (width 0.5) (layer F.Cu) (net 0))
 (segment (start 65.405 86.995) (end 66.015865 86.384135) (width 0.5) (layer F.Cu) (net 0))
 (segment (start 68.5 63.5) (end 69.85 63.5) (width 0.5) (layer F.Cu) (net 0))
 (segment (start 64.77 67.29) (end 59.69 67.29) (width 0.5) (layer F.Cu) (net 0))
 (segment (start 72.39 81.28) (end 68.58 85.09) (width 0.5) (layer F.Cu) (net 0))
 (segment (start 69.85 69.85) (end 71.55 69.85) (width 0.5) (layer F.Cu) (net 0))
 (segment (start 66.015865 86.384135) (end 66.015865 85.059641) (width 0.5) (layer F.Cu) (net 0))
 (segment (start 67.865 62.865) (end 68.5 63.5) (width 0.5) (layer F.Cu) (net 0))
 (segment (start 69.85 74.93) (end 67.31 74.93) (width 0.5) (layer F.Cu) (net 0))
 (segment (start 67.31 64.79) (end 64.77 64.79) (width 0.5) (layer F.Cu) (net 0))
 (segment (start 57.15 78.74) (end 57.15 74.93) (width 0.5) (layer F.Cu) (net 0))
 (segment (start 57.99 74.93) (end 59.69 74.93) (width 0.5) (layer F.Cu) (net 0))
 (segment (start 60.96 67.29) (end 63.5 67.29) (width 0.5) (layer F.Cu) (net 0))
 (segment (start 63.515865 73.675865) (end 62.23 72.39) (width 0.5) (layer F.Cu) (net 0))
 (segment (start 68.58 85.09) (end 68.549641 85.059641) (width 0.5) (layer F.Cu) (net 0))
 (segment (start 63.515865 79.979641) (end 60.970359 79.979641) (width 0.5) (layer F.Cu) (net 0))
 (segment (start 60.96 82.53) (end 58.44 82.53) (width 0.5) (layer F.Cu) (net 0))
 (segment (start 71.2 63.5) (end 69.85 63.5) (width 0.5) (layer F.Cu) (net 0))
 (segment (start 62.23 72.39) (end 59.69 72.39) (width 0.5) (layer F.Cu) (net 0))
 (segment (start 66.015865 76.224135) (end 66.015865 79.979641) (width 0.5) (layer F.Cu) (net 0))
 (segment (start 68.549641 85.059641) (end 66.015865 85.059641) (width 0.5) (layer F.Cu) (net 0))
 (segment (start 58.975 86.995) (end 65.405 86.995) (width 0.5) (layer F.Cu) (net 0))
 (segment (start 63.515865 82.519641) (end 63.515865 85.059641) (width 0.5) (layer F.Cu) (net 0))
 (segment (start 60.970359 79.979641) (end 60.94 80.01) (width 0.5) (layer F.Cu) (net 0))
 (segment (start 58.44 82.53) (end 58.42 82.55) (width 0.5) (layer F.Cu) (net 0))
 (segment (start 58.42 80.01) (end 57.15 78.74) (width 0.5) (layer F.Cu) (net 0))
 (segment (start 58.42 86.44) (end 58.975 86.995) (width 0.5) (layer F.Cu) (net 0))
 (segment (start 67.31 74.93) (end 66.015865 76.224135) (width 0.5) (layer F.Cu) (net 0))
 (segment (start 72.39 64.69) (end 71.2 63.5) (width 0.5) (layer F.Cu) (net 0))
 (segment (start 69.215 67.31) (end 69.195 67.29) (width 0.5) (layer F.Cu) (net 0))
 (segment (start 57.15 73.66) (end 57.15 65.405) (width 0.5) (layer F.Cu) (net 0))
 (segment (start 63.5 62.865) (end 62.865 62.865) (width 0.5) (layer F.Cu) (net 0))
 (segment (start 64.77 69.85) (end 64.77 67.29) (width 0.5) (layer F.Cu) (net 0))
 (segment (start 69.85 72.39) (end 67.31 72.39) (width 0.5) (layer F.Cu) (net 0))
 (segment (start 63.5 62.865) (end 67.865 62.865) (width 0.5) (layer F.Cu) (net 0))
 (segment (start 69.195 67.29) (end 67.945 67.29) (width 0.5) (layer F.Cu) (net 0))
 (segment (start 57.765 64.79) (end 59.69 64.79) (width 0.5) (layer F.Cu) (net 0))
 (segment (start 63.515865 79.979641) (end 63.515865 73.675865) (width 0.5) (layer F.Cu) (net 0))
 (segment (start 62.865 62.865) (end 62.23 63.5) (width 0.5) (layer F.Cu) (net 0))
 (segment (start 67.31 72.39) (end 64.77 69.85) (width 0.5) (layer F.Cu) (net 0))
 (segment (start 70.485 66.04) (end 69.215 67.31) (width 0.5) (layer F.Cu) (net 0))
 (segment (start 57.15 65.405) (end 57.765 64.79) (width 0.5) (layer F.Cu) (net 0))
 (segment (start 72.39 69.85) (end 72.39 64.69) (width 0.5) (layer F.Cu) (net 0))
 (segment (start 57.15 74.93) (end 57.15 73.66) (width 0.5) (layer F.Cu) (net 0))
 (segment (start 69.85 69.85) (end 72.39 69.85) (width 0.5) (layer F.Cu) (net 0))
 (segment (start 72.39 70.69) (end 72.39 69.85) (width 0.5) (layer F.Cu) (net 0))
 (segment (start 57.15 74.93) (end 59.69 74.93) (width 0.5) (layer F.Cu) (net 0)))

